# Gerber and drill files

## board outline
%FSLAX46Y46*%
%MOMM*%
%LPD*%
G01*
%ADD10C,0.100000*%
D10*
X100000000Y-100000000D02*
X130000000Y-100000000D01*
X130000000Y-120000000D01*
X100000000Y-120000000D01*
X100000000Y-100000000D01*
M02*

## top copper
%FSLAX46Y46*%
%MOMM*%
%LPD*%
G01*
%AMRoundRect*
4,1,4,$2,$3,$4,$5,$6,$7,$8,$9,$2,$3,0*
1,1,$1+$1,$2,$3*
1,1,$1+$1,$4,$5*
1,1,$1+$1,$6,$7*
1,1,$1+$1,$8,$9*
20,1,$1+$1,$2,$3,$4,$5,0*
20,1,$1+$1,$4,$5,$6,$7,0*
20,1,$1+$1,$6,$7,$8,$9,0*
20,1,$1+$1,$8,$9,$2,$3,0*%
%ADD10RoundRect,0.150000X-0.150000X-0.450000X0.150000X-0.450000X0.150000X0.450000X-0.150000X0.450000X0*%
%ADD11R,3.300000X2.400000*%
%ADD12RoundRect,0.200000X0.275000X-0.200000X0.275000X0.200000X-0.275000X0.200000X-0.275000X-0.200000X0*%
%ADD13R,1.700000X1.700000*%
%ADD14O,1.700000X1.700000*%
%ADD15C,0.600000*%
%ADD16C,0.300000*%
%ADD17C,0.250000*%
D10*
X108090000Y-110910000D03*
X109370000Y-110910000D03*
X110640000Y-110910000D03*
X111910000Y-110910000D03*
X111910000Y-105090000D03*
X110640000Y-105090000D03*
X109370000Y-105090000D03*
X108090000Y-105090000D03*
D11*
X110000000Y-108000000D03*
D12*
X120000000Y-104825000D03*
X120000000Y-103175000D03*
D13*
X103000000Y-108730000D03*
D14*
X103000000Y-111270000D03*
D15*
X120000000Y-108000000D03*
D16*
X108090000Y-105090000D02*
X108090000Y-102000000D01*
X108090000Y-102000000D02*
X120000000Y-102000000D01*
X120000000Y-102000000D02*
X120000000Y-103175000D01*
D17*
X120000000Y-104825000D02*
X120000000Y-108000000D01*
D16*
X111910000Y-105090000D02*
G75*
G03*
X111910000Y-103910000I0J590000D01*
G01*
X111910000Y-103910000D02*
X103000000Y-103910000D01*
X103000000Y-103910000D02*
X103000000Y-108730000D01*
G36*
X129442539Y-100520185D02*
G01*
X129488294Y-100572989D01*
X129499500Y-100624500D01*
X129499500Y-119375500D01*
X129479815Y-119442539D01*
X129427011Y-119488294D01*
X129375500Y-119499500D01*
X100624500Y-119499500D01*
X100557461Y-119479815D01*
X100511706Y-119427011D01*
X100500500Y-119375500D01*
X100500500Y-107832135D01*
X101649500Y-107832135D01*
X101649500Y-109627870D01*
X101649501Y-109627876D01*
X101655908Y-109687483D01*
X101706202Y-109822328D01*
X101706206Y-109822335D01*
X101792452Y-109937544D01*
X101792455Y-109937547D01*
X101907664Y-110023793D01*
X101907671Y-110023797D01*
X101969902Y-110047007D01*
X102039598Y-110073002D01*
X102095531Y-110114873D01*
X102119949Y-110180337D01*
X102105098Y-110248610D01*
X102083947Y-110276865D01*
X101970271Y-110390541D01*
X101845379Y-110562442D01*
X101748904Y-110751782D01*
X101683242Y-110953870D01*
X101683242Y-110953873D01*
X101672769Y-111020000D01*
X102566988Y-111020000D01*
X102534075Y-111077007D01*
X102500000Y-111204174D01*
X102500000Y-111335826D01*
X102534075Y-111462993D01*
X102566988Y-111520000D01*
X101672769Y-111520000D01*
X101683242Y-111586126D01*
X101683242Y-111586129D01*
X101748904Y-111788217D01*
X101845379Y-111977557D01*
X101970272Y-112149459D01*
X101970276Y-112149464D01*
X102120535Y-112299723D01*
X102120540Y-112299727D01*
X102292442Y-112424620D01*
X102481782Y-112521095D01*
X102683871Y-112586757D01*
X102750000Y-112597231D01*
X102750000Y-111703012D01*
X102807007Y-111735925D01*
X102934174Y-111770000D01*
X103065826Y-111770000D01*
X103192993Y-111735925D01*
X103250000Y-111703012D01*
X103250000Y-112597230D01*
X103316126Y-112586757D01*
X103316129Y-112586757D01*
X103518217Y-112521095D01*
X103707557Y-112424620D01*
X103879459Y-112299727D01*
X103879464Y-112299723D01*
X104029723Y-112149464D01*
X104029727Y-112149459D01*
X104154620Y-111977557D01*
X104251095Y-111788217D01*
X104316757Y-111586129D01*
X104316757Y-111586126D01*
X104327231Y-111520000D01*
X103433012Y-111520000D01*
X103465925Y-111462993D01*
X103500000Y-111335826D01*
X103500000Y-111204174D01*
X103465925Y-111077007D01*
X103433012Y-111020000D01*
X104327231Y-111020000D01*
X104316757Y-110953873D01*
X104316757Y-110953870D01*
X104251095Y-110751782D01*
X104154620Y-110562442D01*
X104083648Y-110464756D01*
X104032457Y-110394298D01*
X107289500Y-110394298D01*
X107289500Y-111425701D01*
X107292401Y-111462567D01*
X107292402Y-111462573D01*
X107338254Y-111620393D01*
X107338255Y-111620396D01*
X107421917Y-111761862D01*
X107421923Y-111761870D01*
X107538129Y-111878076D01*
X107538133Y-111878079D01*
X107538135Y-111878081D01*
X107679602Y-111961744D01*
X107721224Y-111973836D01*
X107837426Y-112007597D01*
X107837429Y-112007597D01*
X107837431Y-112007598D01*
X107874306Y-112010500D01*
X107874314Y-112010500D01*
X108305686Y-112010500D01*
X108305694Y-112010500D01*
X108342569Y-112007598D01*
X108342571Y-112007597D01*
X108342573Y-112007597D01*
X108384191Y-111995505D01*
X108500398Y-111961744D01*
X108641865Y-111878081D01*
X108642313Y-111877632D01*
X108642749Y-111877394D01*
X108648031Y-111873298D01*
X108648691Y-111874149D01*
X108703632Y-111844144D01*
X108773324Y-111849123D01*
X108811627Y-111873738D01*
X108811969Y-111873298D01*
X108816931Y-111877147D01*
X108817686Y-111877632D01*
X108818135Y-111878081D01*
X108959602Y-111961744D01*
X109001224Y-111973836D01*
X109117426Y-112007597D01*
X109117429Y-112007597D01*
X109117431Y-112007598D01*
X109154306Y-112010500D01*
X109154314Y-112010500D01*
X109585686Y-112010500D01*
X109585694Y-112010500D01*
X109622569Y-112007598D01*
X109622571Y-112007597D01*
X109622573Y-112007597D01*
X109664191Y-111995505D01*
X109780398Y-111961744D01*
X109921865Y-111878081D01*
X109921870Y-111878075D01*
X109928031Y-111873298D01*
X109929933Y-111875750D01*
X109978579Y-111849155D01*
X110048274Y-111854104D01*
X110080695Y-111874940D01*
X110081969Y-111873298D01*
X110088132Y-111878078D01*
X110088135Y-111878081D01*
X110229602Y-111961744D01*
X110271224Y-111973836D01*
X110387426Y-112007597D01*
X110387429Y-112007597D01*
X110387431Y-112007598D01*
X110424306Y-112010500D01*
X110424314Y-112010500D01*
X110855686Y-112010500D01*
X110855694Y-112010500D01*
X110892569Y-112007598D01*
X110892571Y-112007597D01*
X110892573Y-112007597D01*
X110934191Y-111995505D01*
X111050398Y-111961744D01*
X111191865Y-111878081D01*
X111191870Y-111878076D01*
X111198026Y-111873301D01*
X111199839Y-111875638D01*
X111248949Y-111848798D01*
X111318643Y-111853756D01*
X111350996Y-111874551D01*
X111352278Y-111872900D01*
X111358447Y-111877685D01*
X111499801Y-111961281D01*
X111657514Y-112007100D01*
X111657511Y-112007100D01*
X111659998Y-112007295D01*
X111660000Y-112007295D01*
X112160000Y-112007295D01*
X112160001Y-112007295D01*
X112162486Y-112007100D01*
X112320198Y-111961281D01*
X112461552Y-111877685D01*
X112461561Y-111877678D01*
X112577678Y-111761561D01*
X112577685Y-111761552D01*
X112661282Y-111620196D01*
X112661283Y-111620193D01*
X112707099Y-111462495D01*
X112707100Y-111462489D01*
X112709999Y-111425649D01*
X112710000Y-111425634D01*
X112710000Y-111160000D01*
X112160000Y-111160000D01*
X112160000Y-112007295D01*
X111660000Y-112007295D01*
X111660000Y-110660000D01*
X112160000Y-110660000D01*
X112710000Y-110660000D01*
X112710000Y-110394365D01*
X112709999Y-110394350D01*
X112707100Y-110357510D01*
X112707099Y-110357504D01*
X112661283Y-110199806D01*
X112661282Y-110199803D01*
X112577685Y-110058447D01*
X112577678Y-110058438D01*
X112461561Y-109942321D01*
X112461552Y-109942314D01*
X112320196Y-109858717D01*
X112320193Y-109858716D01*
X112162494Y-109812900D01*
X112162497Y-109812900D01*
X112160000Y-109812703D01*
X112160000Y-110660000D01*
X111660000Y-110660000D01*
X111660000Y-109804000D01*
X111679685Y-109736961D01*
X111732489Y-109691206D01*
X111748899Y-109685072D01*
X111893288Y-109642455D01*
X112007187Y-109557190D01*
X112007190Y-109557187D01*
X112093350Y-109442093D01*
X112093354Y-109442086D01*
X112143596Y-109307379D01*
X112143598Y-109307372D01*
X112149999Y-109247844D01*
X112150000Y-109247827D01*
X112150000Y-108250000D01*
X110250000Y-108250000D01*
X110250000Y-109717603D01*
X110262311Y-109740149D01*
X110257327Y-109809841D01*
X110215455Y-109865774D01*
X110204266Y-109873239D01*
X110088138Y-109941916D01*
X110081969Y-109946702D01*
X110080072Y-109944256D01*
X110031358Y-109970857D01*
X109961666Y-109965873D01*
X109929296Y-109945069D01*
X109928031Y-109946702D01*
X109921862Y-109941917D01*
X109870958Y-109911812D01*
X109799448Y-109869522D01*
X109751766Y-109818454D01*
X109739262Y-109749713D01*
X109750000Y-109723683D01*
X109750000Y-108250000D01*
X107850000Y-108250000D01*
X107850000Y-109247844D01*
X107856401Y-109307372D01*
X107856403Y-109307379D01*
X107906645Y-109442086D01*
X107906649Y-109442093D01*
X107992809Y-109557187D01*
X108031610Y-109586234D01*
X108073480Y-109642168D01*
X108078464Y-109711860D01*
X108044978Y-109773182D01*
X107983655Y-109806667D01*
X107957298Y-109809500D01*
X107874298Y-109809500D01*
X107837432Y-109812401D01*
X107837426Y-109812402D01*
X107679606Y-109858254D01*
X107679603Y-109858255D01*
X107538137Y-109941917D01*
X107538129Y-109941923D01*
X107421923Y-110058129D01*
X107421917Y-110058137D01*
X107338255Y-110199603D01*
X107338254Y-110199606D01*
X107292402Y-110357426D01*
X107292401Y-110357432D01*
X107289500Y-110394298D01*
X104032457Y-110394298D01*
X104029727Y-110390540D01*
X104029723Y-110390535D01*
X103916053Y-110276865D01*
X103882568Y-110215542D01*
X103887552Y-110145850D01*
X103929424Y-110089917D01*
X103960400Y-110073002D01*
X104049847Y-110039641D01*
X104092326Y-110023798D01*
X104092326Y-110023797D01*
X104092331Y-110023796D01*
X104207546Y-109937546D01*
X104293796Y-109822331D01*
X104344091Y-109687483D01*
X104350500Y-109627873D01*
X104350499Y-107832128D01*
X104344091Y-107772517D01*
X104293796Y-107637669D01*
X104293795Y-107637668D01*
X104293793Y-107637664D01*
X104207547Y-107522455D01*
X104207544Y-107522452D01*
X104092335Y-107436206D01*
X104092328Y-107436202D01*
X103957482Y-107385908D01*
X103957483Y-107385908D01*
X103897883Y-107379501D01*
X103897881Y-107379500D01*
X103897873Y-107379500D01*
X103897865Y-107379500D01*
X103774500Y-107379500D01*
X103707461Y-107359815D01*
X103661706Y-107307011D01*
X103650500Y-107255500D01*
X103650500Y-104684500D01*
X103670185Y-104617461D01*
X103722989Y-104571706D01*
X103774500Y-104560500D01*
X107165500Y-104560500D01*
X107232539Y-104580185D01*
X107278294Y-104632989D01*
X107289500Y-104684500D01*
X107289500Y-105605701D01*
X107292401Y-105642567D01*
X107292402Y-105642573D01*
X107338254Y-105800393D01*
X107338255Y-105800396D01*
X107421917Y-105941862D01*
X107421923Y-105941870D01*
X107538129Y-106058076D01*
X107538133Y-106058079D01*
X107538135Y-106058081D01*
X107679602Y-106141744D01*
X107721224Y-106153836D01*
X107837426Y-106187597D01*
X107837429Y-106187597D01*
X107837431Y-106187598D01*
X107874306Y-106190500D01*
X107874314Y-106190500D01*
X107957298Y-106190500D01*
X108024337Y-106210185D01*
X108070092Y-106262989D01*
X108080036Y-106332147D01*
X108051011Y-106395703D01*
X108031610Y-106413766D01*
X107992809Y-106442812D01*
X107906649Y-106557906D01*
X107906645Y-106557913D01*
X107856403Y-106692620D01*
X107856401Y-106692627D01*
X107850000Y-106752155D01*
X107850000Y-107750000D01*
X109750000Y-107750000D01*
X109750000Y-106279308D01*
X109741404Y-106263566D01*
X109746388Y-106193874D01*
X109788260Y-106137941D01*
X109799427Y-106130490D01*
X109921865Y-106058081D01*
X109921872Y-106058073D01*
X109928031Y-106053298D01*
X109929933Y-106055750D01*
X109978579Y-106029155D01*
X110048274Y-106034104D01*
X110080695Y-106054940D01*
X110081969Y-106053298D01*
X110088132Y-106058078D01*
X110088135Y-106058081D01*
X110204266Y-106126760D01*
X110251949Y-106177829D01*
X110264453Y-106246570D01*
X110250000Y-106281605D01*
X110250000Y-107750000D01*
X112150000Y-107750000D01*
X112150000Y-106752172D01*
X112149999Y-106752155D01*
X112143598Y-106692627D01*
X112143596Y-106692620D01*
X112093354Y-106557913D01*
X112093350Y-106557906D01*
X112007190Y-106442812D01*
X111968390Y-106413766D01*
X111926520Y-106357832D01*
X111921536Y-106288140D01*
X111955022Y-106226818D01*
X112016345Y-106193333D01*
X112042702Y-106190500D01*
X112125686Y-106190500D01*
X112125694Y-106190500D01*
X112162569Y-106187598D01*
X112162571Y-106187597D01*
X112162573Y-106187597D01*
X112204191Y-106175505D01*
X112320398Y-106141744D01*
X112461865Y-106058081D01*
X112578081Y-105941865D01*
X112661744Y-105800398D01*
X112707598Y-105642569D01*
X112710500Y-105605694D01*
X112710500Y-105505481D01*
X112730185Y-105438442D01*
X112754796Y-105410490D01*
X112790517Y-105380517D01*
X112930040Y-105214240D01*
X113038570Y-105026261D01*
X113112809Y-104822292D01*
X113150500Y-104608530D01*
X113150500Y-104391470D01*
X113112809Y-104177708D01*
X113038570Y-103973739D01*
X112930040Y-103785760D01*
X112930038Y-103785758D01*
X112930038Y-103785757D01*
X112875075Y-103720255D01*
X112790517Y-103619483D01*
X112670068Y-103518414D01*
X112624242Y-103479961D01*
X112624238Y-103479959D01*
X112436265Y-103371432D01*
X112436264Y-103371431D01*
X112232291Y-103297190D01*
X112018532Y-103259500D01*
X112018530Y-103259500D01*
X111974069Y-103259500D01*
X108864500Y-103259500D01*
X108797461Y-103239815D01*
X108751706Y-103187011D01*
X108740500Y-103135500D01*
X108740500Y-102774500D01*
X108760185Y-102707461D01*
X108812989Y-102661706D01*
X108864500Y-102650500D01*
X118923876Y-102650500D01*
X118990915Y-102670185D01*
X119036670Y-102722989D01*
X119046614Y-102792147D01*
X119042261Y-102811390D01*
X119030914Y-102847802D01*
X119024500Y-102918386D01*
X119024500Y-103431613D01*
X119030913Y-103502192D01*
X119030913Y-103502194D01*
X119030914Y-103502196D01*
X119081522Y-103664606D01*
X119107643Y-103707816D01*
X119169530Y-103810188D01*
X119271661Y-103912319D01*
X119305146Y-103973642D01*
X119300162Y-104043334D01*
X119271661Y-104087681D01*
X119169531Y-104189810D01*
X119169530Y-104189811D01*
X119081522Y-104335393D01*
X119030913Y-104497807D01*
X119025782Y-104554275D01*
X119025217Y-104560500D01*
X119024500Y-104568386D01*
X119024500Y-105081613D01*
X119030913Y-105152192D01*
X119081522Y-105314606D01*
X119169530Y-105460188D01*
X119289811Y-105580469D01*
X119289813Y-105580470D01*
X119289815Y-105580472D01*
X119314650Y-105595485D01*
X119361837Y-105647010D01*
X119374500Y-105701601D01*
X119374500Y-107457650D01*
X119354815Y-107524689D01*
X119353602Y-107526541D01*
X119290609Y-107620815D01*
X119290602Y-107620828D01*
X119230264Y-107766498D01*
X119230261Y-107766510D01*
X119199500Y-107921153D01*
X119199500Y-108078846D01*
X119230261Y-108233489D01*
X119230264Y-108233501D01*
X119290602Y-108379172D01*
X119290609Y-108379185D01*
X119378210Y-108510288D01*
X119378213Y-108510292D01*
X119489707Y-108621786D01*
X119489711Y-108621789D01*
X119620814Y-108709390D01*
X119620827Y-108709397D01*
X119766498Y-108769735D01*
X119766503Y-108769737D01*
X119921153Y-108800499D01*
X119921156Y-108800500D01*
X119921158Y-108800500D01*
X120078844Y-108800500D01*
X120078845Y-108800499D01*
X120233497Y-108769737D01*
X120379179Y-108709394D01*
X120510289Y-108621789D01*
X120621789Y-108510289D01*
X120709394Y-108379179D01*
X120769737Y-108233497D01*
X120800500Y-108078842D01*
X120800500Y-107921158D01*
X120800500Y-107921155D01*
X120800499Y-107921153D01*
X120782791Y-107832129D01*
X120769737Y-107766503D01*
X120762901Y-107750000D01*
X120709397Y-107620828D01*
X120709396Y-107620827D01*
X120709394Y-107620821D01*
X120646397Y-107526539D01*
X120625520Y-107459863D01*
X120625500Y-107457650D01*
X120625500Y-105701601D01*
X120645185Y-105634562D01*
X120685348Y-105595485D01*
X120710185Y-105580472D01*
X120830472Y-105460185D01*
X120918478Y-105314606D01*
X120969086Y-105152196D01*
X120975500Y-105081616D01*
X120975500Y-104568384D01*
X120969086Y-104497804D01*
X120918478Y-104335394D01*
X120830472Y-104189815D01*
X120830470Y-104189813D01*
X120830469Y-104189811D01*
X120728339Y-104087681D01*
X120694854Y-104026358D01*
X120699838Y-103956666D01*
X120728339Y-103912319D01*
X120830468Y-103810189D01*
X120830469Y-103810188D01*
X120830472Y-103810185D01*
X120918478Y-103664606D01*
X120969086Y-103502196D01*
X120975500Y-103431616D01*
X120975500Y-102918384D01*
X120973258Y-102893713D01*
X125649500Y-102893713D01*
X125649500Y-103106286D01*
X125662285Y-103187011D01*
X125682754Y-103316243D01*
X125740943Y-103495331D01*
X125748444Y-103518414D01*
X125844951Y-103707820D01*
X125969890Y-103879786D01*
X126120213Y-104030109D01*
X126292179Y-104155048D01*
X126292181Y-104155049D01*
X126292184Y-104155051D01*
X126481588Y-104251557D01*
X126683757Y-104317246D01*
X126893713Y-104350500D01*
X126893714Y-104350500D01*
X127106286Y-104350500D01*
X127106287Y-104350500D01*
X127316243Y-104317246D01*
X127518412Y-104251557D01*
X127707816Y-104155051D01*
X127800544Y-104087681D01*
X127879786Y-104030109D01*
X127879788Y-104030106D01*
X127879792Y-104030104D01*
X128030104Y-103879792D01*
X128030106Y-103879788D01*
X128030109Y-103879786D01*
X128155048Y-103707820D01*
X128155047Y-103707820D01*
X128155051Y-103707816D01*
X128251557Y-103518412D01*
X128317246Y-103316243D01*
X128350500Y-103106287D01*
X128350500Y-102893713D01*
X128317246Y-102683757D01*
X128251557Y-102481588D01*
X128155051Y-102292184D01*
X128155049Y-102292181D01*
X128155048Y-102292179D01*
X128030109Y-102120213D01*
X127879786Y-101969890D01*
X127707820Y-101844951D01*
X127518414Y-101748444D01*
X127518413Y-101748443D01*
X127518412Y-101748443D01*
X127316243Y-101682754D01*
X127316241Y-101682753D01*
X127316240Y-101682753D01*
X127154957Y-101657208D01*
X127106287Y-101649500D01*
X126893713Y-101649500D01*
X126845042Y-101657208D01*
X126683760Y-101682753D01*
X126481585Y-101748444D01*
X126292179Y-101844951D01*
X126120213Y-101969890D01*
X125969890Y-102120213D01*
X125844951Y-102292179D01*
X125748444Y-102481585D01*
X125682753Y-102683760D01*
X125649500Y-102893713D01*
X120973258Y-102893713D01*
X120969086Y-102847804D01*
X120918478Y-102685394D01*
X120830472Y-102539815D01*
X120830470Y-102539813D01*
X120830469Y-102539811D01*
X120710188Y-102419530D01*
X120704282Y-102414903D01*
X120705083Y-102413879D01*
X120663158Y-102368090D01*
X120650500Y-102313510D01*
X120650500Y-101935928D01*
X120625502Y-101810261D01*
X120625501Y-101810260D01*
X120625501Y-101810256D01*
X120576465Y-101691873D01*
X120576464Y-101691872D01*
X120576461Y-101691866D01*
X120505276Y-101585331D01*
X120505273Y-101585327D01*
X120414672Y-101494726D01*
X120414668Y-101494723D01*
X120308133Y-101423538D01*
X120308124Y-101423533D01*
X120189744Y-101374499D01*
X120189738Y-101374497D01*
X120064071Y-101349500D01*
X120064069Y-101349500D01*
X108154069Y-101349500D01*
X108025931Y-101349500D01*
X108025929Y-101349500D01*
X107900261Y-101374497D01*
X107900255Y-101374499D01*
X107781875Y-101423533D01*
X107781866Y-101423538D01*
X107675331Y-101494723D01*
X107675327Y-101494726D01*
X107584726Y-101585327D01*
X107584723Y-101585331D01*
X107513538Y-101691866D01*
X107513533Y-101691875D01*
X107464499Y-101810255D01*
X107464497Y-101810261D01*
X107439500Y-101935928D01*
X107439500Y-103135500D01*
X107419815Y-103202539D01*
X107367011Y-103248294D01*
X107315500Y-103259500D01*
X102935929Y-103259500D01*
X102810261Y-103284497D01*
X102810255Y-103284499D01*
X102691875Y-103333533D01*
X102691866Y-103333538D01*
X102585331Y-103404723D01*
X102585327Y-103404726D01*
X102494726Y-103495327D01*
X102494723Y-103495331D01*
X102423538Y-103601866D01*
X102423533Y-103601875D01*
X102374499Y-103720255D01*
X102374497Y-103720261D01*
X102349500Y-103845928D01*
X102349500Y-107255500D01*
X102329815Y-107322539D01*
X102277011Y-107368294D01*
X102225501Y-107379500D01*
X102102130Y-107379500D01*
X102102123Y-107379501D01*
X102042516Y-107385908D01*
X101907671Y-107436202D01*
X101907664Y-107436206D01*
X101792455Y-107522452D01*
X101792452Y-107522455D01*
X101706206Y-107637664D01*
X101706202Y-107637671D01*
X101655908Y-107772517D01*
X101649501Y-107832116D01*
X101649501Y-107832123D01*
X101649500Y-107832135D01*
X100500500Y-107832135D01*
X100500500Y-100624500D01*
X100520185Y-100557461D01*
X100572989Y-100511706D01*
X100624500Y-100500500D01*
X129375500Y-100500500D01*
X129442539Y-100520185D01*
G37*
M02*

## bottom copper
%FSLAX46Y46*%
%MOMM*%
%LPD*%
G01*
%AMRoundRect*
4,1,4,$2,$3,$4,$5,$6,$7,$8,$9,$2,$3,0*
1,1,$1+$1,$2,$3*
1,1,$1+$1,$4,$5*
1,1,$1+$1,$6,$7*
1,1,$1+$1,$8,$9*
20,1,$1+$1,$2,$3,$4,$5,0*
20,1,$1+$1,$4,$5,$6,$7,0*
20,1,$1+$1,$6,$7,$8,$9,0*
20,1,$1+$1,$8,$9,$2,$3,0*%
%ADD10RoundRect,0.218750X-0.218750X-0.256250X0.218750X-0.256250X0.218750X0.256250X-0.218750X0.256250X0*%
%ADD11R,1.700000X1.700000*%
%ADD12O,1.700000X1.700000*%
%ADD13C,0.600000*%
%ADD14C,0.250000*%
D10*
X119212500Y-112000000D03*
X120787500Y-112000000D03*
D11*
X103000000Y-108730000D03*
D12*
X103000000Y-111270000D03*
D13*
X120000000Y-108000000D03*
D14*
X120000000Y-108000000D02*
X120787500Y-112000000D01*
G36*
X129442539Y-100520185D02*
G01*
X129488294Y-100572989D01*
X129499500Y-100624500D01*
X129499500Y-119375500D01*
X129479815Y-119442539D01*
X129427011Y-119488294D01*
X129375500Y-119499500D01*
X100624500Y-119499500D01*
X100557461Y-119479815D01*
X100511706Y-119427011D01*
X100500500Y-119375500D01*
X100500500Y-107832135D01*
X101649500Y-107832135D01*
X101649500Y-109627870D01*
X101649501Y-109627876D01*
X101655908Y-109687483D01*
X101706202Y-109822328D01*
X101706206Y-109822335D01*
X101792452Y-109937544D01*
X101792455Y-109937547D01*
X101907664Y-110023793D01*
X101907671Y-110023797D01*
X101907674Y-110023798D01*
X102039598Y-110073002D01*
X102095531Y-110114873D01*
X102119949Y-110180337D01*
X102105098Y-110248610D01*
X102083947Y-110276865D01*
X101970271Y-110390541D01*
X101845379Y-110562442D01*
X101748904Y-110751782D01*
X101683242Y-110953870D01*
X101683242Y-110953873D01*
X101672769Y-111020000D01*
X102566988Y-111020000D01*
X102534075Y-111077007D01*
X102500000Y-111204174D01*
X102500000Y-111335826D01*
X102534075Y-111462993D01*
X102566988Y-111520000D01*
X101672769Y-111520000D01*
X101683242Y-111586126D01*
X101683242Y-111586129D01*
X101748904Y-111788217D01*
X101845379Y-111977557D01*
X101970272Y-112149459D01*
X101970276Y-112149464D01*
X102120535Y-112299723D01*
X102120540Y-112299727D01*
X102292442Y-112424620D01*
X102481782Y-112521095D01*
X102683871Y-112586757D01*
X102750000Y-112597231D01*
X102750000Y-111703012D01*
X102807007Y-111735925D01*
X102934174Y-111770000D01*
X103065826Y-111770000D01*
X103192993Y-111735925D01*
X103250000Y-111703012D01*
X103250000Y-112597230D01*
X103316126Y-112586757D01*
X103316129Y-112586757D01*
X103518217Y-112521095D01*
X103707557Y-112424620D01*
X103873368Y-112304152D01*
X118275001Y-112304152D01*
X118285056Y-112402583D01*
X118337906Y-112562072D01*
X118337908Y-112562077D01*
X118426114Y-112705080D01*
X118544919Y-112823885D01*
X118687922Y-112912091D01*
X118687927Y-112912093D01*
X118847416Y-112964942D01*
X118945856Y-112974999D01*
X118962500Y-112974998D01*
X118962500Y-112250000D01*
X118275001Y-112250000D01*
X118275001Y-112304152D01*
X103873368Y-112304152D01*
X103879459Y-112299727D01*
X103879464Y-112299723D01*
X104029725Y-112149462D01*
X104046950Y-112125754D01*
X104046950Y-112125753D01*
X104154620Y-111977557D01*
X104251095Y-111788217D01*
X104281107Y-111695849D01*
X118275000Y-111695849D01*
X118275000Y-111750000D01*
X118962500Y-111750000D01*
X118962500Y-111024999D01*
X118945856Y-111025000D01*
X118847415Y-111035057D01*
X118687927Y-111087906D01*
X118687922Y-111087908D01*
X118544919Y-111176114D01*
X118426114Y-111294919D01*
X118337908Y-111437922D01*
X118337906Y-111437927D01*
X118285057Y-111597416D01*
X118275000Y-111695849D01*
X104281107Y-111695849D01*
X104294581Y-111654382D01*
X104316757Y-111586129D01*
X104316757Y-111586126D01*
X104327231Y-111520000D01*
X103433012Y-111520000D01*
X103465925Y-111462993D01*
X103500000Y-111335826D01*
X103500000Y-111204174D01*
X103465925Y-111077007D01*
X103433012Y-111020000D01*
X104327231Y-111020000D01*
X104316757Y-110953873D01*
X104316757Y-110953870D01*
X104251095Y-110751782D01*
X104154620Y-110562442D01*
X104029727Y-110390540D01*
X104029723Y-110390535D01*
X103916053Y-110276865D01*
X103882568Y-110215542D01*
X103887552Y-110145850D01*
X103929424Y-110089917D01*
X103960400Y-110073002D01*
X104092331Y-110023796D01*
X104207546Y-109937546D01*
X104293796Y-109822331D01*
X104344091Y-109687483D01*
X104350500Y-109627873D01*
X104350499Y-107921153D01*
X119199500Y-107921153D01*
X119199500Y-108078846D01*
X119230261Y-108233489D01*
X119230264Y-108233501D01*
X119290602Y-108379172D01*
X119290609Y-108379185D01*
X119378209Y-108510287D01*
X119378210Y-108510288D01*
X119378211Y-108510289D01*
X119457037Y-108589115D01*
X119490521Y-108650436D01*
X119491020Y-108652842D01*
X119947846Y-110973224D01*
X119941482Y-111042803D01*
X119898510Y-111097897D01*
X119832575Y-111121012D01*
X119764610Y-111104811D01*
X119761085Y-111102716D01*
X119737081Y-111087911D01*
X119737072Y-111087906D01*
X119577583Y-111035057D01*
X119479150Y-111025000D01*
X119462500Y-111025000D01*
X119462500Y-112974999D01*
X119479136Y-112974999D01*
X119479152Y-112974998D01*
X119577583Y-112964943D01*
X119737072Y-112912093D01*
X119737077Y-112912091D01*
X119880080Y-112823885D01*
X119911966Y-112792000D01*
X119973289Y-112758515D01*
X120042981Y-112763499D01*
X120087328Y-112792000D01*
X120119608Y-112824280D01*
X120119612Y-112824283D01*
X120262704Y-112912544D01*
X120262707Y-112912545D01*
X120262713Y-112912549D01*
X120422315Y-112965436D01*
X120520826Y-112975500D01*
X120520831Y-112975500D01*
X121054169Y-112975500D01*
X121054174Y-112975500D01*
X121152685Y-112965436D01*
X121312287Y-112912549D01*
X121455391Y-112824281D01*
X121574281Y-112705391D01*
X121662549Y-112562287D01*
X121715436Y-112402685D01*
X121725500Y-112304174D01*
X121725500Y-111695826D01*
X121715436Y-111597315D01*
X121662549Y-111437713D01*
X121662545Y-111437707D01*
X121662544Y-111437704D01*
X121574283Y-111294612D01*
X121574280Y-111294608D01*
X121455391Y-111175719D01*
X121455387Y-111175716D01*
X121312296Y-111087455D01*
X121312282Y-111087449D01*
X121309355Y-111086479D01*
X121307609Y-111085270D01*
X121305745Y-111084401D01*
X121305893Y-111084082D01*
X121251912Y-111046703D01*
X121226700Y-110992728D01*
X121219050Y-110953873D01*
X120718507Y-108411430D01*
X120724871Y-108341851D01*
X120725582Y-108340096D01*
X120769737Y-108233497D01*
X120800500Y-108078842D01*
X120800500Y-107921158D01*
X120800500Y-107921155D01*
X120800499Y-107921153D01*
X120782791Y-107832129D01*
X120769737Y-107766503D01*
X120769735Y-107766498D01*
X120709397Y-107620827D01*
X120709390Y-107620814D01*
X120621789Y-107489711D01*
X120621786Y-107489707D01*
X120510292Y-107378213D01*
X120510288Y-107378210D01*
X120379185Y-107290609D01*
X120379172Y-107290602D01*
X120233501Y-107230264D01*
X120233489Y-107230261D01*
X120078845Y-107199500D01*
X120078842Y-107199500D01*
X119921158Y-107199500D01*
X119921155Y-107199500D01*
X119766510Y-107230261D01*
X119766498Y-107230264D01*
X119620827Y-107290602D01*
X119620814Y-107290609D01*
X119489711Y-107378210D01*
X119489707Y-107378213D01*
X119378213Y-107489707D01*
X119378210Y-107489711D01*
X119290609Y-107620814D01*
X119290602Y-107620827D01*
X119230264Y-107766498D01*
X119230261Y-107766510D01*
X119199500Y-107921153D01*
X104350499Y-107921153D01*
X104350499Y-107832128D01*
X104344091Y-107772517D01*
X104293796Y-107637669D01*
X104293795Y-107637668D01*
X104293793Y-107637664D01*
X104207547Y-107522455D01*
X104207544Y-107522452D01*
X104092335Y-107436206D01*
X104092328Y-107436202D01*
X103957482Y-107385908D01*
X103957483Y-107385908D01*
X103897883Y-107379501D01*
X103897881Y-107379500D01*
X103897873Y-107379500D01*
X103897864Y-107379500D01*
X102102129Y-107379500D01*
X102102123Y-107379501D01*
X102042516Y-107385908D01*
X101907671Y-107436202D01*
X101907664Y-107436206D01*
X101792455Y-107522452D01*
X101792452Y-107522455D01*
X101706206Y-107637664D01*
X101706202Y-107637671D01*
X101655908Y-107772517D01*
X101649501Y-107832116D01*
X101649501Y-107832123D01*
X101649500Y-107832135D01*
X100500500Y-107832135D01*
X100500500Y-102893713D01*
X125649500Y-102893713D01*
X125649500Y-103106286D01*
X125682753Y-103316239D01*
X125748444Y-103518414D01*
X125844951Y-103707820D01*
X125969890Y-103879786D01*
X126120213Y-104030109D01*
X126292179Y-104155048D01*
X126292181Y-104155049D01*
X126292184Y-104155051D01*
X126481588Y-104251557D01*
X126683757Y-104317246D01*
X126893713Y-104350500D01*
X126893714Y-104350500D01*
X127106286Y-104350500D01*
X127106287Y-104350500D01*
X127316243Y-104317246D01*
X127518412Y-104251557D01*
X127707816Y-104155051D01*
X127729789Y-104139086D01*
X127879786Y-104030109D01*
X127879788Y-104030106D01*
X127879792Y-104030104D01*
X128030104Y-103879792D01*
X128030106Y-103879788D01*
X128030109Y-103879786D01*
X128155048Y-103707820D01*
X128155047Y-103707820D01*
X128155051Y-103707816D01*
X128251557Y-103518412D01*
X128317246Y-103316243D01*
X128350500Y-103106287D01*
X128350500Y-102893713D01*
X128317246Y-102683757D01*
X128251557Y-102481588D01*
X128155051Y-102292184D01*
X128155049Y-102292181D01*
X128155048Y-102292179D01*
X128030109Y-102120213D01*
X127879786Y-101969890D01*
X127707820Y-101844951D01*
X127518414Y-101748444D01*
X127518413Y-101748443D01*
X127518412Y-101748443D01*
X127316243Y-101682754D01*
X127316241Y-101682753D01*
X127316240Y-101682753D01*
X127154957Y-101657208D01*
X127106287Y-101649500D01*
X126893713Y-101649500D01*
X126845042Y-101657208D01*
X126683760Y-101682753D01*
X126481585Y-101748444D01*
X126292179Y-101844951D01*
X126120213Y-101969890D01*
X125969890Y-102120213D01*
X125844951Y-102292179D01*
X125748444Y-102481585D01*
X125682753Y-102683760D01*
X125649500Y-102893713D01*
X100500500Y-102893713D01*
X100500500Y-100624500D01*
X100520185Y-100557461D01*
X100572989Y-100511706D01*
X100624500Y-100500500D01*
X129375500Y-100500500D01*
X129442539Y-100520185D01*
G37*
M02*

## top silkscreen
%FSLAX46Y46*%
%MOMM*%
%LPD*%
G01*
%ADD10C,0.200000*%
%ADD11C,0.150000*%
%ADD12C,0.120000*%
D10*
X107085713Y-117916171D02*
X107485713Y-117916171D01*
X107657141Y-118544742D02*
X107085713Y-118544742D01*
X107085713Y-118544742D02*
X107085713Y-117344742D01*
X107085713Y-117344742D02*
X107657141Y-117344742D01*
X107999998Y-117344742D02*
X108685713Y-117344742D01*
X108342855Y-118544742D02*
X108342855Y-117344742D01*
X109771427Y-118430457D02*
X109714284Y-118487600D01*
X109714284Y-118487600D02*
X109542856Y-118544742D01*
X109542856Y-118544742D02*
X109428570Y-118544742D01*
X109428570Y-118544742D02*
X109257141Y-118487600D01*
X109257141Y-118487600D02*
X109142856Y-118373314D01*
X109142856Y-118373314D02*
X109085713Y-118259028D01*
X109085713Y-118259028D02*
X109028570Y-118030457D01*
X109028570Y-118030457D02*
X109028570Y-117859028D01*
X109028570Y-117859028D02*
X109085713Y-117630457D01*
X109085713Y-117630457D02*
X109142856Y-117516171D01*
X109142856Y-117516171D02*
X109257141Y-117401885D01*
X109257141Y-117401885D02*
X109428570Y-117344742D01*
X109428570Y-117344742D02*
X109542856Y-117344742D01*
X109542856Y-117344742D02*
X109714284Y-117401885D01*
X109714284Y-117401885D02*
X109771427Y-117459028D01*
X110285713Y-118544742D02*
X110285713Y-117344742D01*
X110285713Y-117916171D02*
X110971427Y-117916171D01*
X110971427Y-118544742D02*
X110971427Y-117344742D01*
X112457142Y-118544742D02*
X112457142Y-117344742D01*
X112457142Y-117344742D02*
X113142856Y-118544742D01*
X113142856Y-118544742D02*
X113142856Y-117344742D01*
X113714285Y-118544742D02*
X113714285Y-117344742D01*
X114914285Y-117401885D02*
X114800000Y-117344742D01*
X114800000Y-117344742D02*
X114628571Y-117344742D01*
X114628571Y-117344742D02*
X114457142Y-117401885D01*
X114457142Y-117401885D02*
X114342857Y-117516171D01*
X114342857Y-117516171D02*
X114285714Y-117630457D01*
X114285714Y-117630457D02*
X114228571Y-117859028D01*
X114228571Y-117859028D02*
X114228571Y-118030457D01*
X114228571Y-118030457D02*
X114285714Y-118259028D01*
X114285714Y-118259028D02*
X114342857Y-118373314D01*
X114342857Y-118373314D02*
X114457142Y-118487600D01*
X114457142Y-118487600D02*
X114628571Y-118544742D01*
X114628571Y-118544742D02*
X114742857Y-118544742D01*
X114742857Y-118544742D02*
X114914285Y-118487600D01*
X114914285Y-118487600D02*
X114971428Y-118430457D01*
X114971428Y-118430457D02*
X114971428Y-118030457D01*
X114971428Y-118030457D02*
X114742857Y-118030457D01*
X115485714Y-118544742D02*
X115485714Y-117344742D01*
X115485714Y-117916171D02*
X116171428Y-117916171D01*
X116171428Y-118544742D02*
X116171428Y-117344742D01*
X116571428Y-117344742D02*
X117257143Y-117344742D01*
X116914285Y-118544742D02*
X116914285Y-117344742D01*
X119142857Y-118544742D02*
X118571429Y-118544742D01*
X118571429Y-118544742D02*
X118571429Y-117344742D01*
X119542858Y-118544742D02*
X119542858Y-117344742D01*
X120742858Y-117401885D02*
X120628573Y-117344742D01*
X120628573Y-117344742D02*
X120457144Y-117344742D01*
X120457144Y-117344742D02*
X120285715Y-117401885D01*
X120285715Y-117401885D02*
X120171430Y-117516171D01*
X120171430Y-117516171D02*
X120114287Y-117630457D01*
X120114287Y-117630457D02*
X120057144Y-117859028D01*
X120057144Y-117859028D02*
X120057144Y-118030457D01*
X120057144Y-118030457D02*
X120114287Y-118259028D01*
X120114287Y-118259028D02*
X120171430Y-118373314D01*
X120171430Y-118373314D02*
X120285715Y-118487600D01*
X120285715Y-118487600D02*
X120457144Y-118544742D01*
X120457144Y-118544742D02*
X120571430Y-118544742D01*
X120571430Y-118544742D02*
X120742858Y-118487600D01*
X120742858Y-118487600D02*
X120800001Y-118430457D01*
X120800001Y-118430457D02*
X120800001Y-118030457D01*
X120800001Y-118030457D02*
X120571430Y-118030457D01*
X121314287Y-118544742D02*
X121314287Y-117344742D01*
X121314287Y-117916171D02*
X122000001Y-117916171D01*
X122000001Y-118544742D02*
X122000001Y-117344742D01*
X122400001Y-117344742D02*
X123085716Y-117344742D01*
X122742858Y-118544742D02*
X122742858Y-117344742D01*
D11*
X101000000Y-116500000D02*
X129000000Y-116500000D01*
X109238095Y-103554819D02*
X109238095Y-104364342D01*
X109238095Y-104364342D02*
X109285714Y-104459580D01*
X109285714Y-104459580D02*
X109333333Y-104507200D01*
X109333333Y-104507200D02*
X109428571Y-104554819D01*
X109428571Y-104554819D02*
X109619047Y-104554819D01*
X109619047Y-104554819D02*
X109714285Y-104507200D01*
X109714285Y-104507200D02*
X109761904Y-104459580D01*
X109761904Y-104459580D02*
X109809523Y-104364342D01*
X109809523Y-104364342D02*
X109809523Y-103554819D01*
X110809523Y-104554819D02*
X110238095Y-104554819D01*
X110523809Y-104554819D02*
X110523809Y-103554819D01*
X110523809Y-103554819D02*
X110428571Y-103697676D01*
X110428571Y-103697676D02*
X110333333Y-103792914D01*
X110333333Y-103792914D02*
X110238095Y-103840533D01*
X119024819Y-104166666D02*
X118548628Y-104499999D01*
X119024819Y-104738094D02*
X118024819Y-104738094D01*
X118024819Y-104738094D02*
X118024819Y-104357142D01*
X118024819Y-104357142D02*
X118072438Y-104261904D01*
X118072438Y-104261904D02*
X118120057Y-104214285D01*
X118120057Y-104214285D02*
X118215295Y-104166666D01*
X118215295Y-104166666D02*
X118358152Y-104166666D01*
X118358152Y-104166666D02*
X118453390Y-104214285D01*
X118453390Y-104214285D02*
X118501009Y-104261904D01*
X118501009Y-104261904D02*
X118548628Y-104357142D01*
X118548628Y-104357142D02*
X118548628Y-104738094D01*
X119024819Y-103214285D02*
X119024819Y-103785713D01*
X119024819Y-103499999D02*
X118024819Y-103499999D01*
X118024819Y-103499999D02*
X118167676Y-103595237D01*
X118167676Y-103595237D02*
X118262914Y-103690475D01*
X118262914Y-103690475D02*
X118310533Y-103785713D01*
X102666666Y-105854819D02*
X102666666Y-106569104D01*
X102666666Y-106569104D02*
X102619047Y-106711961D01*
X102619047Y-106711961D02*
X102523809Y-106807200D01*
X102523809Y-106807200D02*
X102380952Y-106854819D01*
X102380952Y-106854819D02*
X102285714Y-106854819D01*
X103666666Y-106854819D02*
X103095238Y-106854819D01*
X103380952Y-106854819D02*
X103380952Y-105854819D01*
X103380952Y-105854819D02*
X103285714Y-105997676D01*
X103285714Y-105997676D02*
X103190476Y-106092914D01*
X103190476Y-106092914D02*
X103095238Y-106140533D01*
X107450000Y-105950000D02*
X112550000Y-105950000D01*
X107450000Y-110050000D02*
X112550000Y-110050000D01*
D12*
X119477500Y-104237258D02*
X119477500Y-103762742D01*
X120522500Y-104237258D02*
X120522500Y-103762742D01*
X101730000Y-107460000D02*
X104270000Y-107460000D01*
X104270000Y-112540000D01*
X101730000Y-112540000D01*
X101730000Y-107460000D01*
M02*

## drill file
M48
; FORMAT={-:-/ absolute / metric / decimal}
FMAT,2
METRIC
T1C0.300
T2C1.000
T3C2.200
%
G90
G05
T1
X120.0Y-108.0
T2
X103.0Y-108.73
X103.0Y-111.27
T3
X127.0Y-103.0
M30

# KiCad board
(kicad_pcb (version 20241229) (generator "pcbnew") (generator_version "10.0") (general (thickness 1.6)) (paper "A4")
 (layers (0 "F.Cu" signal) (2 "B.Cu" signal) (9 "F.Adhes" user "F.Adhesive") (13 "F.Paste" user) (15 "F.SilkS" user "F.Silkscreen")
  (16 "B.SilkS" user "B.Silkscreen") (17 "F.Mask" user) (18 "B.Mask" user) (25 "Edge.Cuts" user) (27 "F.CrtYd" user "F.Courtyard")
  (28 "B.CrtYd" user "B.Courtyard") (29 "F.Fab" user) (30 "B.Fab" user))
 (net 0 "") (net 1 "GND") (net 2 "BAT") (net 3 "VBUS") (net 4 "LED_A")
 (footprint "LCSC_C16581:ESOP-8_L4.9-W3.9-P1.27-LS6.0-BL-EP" (layer "F.Cu") (at 110 108)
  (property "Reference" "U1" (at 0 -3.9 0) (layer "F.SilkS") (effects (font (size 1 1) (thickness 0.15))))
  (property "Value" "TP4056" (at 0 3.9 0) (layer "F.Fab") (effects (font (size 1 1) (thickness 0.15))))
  (fp_line (start -2.55 -2.05) (end 2.55 -2.05) (stroke (width 0.15) (type default)) (layer "F.SilkS"))
  (fp_line (start -2.55 2.05) (end 2.55 2.05) (stroke (width 0.15) (type default)) (layer "F.SilkS"))
  (pad "1" smd roundrect (at -1.91 2.91) (size 0.6 1.2) (layers "F.Cu" "F.Paste" "F.Mask") (roundrect_rratio 0.25) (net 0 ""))
  (pad "2" smd roundrect (at -0.63 2.91) (size 0.6 1.2) (layers "F.Cu" "F.Paste" "F.Mask") (roundrect_rratio 0.25) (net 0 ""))
  (pad "3" smd roundrect (at 0.64 2.91) (size 0.6 1.2) (layers "F.Cu" "F.Paste" "F.Mask") (roundrect_rratio 0.25) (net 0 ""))
  (pad "4" smd roundrect (at 1.91 2.91) (size 0.6 1.2) (layers "F.Cu" "F.Paste" "F.Mask") (roundrect_rratio 0.25) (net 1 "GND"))
  (pad "5" smd roundrect (at 1.91 -2.91) (size 0.6 1.2) (layers "F.Cu" "F.Paste" "F.Mask") (roundrect_rratio 0.25) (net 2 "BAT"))
  (pad "6" smd roundrect (at 0.64 -2.91) (size 0.6 1.2) (layers "F.Cu" "F.Paste" "F.Mask") (roundrect_rratio 0.25) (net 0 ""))
  (pad "7" smd roundrect (at -0.63 -2.91) (size 0.6 1.2) (layers "F.Cu" "F.Paste" "F.Mask") (roundrect_rratio 0.25) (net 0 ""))
  (pad "8" smd roundrect (at -1.91 -2.91) (size 0.6 1.2) (layers "F.Cu" "F.Paste" "F.Mask") (roundrect_rratio 0.25) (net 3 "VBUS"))
  (pad "9" smd rect (at 0 0 180) (size 3.3 2.4) (layers "F.Cu" "F.Paste" "F.Mask") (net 1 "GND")))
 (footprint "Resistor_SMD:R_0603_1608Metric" (layer "F.Cu") (at 120 104 90)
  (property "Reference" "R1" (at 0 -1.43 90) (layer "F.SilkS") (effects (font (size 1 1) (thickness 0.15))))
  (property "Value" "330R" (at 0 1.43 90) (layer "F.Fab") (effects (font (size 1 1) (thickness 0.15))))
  (fp_line (start -0.237258 -0.5225) (end 0.237258 -0.5225) (stroke (width 0.12) (type solid)) (layer "F.SilkS"))
  (fp_line (start -0.237258 0.5225) (end 0.237258 0.5225) (stroke (width 0.12) (type solid)) (layer "F.SilkS"))
  (pad "1" smd roundrect (at -0.825 0 90) (size 0.8 0.95) (layers "F.Cu" "F.Paste" "F.Mask") (roundrect_rratio 0.25) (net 3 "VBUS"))
  (pad "2" smd roundrect (at 0.825 0 90) (size 0.8 0.95) (layers "F.Cu" "F.Paste" "F.Mask") (roundrect_rratio 0.25) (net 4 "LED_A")))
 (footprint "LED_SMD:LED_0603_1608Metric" (layer "B.Cu") (at 120 112)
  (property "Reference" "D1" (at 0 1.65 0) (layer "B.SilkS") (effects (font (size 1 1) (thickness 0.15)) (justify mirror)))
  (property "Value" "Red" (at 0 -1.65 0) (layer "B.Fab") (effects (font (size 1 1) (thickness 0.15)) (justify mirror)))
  (pad "1" smd roundrect (at -0.7875 0) (size 0.875 0.95) (layers "B.Cu" "B.Paste" "B.Mask") (roundrect_rratio 0.25) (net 1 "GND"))
  (pad "2" smd roundrect (at 0.7875 0) (size 0.875 0.95) (layers "B.Cu" "B.Paste" "B.Mask") (roundrect_rratio 0.25) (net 4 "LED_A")))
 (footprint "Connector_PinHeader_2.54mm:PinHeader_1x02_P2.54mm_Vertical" (layer "F.Cu") (at 103 108.73)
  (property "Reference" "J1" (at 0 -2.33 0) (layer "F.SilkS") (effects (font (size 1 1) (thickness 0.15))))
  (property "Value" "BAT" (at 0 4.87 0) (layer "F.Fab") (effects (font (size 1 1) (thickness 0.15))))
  (fp_rect (start -1.27 -1.27) (end 1.27 3.81) (stroke (width 0.12) (type solid)) (layer "F.SilkS"))
  (pad "1" thru_hole rect (at 0 0) (size 1.7 1.7) (drill 1) (layers "*.Cu" "*.Mask") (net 2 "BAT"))
  (pad "2" thru_hole oval (at 0 2.54) (size 1.7 1.7) (drill 1) (layers "*.Cu" "*.Mask") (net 1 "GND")))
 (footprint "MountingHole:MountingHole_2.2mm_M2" (layer "F.Cu") (at 127 103)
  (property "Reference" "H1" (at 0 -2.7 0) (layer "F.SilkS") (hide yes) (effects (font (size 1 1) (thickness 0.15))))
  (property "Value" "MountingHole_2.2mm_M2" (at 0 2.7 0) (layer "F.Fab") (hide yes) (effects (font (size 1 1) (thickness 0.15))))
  (pad "" np_thru_hole circle (at 0 0) (size 2.2 2.2) (drill 2.2) (layers "*.Cu" "*.Mask")))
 (gr_rect (start 100 100) (end 130 120) (stroke (width 0.1) (type default)) (fill no) (layer "Edge.Cuts"))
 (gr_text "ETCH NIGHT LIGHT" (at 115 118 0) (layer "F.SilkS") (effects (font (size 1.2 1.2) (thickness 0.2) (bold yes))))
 (gr_line (start 101 116.5) (end 129 116.5) (stroke (width 0.15) (type default)) (layer "F.SilkS"))
 (segment (start 108.09 105.09) (end 108.09 102) (width 0.3) (layer "F.Cu") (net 3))
 (segment (start 108.09 102) (end 120 102) (width 0.3) (layer "F.Cu") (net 3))
 (segment (start 120 102) (end 120 103.175) (width 0.3) (layer "F.Cu") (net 3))
 (segment (start 120 104.825) (end 120 108) (width 0.25) (layer "F.Cu") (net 4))
 (via (at 120 108) (size 0.6) (drill 0.3) (layers "F.Cu" "B.Cu") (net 4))
 (segment (start 120 108) (end 120.7875 112) (width 0.25) (layer "B.Cu") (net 4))
 (arc (start 111.91 105.09) (mid 112.5 104.5) (end 111.91 103.91) (width 0.3) (layer "F.Cu") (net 2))
 (segment (start 111.91 103.91) (end 103 103.91) (width 0.3) (layer "F.Cu") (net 2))
 (segment (start 103 103.91) (end 103 108.73) (width 0.3) (layer "F.Cu") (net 2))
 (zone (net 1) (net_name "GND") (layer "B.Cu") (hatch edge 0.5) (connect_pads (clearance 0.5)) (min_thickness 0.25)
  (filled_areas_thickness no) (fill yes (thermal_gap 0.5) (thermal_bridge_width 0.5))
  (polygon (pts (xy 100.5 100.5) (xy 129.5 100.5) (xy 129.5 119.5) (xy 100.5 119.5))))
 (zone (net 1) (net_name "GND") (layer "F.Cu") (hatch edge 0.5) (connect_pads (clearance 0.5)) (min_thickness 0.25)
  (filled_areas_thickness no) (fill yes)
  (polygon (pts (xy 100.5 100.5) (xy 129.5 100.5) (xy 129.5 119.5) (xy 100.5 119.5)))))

